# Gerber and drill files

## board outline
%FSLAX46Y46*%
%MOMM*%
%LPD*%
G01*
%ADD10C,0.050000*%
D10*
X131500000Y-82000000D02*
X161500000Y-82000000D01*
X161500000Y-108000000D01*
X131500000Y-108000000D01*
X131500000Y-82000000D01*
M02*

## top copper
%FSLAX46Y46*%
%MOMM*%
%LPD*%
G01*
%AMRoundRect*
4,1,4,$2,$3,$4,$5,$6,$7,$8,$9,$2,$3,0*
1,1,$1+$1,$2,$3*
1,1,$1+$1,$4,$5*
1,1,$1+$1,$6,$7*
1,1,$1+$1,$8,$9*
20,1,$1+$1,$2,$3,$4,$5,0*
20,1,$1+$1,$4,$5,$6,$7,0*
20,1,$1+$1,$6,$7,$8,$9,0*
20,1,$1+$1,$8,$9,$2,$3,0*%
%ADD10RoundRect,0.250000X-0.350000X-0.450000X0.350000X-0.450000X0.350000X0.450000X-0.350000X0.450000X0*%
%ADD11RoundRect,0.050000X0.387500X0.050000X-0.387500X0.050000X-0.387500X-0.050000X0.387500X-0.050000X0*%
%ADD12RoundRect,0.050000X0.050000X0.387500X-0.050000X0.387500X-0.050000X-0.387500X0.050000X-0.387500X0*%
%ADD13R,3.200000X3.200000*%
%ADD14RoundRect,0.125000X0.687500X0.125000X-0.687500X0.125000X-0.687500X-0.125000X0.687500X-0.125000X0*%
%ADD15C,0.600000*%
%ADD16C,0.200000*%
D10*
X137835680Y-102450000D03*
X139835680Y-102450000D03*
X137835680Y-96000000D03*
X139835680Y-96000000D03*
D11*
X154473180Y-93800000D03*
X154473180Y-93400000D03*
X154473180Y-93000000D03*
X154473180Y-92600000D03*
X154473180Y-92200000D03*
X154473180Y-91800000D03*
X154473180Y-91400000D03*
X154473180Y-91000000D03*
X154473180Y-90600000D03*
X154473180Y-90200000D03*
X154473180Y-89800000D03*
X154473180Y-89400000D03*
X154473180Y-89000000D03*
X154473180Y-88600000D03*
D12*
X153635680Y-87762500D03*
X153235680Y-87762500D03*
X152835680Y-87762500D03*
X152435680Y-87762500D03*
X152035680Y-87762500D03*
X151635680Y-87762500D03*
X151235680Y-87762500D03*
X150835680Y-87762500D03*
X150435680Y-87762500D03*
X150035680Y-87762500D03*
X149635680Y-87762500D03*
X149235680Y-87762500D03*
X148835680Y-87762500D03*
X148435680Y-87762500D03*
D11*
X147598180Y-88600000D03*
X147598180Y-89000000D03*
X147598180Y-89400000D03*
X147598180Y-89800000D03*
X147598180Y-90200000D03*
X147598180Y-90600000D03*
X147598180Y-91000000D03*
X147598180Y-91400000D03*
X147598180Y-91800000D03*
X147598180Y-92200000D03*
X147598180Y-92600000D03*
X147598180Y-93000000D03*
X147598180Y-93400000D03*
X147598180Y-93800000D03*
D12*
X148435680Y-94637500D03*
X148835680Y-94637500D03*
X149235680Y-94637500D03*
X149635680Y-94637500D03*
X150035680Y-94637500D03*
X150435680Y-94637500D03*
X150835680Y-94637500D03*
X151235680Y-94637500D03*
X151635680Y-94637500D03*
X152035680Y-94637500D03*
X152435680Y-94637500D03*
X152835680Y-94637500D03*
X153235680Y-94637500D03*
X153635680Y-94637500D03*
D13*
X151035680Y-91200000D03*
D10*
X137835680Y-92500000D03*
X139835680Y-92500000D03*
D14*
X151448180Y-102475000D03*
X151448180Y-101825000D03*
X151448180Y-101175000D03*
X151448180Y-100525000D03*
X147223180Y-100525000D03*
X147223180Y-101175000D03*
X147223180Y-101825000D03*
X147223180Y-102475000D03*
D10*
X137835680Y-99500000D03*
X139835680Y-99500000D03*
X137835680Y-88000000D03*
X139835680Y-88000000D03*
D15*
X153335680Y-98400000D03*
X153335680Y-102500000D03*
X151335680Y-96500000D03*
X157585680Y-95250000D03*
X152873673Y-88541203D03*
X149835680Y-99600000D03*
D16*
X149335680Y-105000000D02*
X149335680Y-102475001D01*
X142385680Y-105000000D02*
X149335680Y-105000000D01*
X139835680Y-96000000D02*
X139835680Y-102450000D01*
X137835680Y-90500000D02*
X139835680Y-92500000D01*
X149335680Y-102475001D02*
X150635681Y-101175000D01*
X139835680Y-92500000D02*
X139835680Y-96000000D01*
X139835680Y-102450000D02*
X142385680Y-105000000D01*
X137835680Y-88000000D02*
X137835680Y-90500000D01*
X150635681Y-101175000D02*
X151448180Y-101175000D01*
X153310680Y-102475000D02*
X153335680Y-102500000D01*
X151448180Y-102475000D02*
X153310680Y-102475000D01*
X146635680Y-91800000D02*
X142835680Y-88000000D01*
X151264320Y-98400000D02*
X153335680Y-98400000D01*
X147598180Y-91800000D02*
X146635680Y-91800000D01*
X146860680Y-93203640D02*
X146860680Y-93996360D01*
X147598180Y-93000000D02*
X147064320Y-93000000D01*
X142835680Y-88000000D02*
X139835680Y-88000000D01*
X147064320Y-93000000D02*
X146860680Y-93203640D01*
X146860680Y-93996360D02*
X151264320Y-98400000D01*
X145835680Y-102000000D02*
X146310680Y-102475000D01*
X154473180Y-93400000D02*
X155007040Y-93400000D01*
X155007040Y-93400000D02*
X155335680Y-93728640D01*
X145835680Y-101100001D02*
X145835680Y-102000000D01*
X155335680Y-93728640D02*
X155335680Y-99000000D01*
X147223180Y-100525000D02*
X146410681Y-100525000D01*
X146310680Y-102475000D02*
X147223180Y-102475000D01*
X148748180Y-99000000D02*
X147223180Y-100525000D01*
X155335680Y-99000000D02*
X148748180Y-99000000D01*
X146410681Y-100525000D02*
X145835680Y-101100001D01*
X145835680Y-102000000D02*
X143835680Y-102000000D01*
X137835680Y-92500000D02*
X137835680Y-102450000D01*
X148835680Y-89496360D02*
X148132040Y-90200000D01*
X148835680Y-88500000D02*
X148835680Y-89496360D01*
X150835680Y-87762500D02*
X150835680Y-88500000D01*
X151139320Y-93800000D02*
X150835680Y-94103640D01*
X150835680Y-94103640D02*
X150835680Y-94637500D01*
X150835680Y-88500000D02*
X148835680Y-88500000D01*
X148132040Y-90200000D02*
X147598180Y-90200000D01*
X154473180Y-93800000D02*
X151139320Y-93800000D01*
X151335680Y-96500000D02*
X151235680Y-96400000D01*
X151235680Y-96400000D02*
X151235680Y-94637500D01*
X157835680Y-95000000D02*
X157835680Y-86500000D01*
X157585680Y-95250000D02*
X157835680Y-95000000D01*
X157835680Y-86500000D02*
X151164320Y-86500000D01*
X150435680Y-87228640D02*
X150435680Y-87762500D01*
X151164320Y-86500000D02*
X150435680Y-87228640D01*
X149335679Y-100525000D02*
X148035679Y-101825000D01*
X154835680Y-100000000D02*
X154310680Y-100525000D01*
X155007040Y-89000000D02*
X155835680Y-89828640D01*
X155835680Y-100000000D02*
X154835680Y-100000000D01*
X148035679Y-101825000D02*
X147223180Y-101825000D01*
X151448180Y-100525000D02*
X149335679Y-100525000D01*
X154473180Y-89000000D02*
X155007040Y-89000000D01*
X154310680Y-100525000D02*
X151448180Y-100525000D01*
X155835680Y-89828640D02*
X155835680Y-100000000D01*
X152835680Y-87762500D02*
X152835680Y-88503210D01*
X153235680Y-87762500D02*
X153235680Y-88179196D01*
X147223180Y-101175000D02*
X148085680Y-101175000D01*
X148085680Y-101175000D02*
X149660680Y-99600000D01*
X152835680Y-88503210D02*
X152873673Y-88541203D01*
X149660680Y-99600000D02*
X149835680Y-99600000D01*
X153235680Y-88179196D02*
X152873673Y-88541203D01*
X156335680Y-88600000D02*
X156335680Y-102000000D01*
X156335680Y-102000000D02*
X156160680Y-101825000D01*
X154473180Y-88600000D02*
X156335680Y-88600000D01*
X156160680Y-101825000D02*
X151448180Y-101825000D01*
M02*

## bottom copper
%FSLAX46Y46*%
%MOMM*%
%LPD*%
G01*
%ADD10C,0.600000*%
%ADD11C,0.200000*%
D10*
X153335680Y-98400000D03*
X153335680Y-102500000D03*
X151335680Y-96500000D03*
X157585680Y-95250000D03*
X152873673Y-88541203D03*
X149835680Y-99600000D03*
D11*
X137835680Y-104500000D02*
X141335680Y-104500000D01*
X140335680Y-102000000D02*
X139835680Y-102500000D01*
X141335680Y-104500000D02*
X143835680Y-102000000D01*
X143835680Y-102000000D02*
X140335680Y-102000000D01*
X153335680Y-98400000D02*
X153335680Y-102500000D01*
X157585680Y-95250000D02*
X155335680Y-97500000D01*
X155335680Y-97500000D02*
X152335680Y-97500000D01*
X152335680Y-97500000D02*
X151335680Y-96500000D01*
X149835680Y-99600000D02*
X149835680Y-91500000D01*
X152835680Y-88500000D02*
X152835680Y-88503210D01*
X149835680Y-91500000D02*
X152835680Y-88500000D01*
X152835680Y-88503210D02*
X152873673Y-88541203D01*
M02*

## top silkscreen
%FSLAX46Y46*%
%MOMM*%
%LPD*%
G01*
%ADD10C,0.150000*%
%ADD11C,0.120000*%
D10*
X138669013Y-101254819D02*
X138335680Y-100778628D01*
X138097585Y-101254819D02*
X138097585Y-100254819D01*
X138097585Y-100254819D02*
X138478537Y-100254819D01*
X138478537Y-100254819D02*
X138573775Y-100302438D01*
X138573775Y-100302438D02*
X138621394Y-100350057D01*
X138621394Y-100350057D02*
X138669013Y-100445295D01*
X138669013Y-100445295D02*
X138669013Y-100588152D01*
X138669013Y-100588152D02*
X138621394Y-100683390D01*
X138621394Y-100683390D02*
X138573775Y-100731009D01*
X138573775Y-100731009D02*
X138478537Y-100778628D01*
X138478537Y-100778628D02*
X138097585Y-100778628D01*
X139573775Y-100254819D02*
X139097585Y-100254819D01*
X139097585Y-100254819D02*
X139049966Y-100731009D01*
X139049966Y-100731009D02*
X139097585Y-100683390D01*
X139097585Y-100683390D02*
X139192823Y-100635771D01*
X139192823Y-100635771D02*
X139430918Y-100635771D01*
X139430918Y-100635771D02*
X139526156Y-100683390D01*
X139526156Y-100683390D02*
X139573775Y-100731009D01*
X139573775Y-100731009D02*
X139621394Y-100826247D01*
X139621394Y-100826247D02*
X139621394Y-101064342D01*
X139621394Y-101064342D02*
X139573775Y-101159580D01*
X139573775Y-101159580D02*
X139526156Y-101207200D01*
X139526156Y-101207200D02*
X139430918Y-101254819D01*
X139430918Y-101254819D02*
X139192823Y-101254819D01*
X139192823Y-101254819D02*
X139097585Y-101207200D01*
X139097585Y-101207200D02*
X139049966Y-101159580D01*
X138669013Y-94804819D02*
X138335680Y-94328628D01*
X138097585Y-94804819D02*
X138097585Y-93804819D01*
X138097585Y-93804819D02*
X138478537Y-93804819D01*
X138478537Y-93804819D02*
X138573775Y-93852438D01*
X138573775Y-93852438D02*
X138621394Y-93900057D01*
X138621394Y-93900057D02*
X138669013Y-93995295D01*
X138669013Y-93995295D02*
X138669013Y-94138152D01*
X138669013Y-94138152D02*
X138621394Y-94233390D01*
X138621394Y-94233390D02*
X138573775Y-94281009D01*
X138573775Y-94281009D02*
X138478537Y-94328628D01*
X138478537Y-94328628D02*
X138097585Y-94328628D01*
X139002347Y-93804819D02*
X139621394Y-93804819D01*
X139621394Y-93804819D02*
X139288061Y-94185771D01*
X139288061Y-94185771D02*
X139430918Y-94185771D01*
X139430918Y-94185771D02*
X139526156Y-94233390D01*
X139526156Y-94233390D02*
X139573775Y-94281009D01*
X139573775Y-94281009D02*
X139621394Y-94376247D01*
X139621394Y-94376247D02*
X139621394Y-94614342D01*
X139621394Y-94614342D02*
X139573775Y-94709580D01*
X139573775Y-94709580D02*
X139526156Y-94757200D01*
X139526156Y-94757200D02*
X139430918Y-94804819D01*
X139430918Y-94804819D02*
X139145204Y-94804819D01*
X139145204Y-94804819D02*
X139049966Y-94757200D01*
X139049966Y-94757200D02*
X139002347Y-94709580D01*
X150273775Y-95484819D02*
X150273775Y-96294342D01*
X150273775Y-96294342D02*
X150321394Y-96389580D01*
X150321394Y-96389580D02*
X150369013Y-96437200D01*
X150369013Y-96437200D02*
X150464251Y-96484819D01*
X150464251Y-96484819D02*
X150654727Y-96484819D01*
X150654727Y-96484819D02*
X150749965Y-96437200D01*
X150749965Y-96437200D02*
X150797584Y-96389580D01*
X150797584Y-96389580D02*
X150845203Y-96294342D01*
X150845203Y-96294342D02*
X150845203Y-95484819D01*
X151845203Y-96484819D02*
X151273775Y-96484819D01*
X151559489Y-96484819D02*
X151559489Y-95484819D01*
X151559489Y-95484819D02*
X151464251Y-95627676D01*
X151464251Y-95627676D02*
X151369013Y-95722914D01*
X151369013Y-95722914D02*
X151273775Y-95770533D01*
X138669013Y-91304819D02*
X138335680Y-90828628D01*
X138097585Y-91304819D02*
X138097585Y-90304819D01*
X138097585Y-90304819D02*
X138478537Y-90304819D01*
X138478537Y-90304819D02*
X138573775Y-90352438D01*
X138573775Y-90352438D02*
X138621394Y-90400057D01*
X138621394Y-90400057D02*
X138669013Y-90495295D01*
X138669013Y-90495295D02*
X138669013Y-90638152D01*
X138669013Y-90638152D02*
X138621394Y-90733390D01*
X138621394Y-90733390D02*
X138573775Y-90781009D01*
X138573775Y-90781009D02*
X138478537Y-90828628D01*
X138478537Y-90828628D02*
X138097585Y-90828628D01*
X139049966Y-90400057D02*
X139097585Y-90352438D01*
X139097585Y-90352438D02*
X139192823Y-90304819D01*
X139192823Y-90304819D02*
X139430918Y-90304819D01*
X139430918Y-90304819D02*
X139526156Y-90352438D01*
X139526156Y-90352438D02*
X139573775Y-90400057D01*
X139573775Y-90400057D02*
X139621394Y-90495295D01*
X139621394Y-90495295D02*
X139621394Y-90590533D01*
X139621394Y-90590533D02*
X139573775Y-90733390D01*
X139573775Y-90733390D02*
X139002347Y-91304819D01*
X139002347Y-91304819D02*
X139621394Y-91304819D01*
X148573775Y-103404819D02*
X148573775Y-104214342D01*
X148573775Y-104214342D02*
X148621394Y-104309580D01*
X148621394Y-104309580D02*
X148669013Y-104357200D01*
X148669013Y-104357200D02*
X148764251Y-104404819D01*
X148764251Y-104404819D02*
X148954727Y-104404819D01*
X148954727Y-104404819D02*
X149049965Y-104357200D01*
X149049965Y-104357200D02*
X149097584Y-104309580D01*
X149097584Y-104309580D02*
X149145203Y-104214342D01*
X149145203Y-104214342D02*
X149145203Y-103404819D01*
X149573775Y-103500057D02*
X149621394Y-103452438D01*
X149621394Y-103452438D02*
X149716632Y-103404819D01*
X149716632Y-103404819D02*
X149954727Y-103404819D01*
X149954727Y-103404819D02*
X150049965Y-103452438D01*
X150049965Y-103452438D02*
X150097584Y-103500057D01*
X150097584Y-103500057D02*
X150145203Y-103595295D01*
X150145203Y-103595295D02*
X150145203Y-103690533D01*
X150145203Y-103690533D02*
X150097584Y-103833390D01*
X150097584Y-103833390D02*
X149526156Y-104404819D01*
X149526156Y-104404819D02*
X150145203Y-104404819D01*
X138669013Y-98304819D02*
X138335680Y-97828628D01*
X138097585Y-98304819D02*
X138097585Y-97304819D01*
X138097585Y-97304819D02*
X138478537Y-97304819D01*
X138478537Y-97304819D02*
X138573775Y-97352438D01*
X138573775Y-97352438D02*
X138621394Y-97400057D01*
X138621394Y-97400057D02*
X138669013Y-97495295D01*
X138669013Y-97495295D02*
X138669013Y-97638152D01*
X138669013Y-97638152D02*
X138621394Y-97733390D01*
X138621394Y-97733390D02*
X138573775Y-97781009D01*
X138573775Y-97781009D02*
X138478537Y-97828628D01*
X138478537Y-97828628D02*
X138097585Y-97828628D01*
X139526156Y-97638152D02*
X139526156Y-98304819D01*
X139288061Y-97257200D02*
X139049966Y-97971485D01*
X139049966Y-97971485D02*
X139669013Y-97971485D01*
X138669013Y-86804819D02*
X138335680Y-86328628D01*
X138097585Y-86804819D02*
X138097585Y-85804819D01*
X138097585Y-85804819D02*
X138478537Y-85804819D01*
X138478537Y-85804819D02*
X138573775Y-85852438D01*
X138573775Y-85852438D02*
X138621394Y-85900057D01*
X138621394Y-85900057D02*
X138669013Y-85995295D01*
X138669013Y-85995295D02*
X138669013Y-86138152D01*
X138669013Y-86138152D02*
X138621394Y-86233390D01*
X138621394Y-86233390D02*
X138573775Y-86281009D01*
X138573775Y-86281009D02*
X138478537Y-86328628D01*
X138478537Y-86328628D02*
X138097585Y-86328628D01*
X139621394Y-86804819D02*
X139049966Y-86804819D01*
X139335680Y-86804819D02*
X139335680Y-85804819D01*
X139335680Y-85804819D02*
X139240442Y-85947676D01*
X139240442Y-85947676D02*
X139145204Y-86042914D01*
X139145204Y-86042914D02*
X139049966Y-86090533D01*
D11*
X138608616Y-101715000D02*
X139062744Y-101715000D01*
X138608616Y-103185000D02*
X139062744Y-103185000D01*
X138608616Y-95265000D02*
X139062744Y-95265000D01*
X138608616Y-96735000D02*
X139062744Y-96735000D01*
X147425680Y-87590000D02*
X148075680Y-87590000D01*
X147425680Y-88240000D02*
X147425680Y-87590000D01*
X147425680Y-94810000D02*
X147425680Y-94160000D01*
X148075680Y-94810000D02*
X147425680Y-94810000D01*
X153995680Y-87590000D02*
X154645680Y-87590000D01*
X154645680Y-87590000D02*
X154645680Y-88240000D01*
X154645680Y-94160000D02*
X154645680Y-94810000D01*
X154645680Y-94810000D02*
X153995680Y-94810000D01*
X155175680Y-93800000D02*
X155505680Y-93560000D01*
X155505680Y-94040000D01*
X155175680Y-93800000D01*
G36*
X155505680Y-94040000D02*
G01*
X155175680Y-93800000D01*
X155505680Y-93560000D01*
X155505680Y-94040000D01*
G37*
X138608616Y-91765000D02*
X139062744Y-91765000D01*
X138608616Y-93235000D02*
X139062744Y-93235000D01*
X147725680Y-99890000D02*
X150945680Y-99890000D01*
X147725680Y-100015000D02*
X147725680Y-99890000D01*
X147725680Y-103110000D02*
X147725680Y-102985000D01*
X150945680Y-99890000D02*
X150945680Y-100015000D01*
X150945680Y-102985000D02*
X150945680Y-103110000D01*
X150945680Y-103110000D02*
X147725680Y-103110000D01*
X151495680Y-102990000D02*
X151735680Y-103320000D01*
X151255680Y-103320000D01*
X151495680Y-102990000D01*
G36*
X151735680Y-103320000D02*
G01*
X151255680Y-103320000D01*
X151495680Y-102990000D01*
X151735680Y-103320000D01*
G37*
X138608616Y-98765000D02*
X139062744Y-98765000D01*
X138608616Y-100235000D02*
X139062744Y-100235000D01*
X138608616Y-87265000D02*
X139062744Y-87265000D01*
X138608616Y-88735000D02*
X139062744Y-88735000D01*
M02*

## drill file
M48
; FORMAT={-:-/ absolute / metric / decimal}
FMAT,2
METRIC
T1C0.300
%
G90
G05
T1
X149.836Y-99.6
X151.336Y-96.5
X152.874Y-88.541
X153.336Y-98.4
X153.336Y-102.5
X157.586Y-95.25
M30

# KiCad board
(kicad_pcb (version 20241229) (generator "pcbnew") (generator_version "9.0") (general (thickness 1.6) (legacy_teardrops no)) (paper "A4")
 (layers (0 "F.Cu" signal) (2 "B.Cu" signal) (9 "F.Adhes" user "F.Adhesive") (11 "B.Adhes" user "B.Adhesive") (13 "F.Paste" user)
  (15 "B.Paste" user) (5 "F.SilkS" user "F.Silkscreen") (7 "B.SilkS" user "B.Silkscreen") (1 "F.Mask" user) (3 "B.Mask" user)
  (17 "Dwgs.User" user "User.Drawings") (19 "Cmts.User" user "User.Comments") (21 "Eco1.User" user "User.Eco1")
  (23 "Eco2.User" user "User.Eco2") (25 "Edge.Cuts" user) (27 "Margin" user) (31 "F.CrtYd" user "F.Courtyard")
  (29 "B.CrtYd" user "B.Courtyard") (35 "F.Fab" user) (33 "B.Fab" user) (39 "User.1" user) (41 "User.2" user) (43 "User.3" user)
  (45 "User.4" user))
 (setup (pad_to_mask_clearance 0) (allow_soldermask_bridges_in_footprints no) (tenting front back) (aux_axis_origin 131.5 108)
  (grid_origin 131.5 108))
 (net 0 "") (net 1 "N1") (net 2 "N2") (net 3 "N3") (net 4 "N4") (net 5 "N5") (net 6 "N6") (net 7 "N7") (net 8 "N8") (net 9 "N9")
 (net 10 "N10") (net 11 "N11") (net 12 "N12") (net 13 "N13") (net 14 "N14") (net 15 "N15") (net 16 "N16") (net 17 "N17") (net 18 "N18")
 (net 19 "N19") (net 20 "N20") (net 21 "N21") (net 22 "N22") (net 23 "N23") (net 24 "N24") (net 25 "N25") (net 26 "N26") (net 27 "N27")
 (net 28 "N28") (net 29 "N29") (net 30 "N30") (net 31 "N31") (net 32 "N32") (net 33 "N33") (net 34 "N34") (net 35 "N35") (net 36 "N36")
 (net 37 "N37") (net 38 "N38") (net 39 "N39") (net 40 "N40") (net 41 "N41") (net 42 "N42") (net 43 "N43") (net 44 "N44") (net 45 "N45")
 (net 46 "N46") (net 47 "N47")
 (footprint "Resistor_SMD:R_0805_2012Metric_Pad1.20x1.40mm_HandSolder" (layer "F.Cu") (at 138.83568 102.45)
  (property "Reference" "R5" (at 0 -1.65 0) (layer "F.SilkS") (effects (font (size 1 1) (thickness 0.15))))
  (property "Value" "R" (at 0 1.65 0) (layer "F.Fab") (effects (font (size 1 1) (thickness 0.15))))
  (fp_line (start -0.227064 -0.735) (end 0.227064 -0.735) (stroke (width 0.12) (type solid)) (layer "F.SilkS"))
  (fp_line (start -0.227064 0.735) (end 0.227064 0.735) (stroke (width 0.12) (type solid)) (layer "F.SilkS"))
  (pad "1" smd roundrect (at -1 0) (size 1.2 1.4) (layers "F.Cu" "F.Mask" "F.Paste") (roundrect_rratio 0.208333) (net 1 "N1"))
  (pad "2" smd roundrect (at 1 0) (size 1.2 1.4) (layers "F.Cu" "F.Mask" "F.Paste") (roundrect_rratio 0.208333) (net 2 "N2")))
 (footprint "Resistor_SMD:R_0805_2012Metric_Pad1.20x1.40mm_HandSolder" (layer "F.Cu") (at 138.83568 96)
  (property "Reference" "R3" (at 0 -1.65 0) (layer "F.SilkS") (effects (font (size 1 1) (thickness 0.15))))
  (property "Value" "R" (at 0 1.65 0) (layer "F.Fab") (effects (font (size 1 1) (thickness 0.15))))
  (fp_line (start -0.227064 -0.735) (end 0.227064 -0.735) (stroke (width 0.12) (type solid)) (layer "F.SilkS"))
  (fp_line (start -0.227064 0.735) (end 0.227064 0.735) (stroke (width 0.12) (type solid)) (layer "F.SilkS"))
  (pad "1" smd roundrect (at -1 0) (size 1.2 1.4) (layers "F.Cu" "F.Mask" "F.Paste") (roundrect_rratio 0.208333) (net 1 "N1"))
  (pad "2" smd roundrect (at 1 0) (size 1.2 1.4) (layers "F.Cu" "F.Mask" "F.Paste") (roundrect_rratio 0.208333) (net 2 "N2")))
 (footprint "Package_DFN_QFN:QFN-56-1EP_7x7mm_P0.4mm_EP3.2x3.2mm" (layer "F.Cu") (at 151.03568 91.2 180)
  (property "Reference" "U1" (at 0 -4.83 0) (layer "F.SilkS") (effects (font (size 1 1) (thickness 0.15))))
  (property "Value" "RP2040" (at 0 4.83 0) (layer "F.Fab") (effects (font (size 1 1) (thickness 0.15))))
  (fp_line (start 3.61 3.61) (end 2.96 3.61) (stroke (width 0.12) (type solid)) (layer "F.SilkS"))
  (fp_line (start 3.61 2.96) (end 3.61 3.61) (stroke (width 0.12) (type solid)) (layer "F.SilkS"))
  (fp_line (start 3.61 -3.61) (end 3.61 -2.96) (stroke (width 0.12) (type solid)) (layer "F.SilkS"))
  (fp_line (start 2.96 -3.61) (end 3.61 -3.61) (stroke (width 0.12) (type solid)) (layer "F.SilkS"))
  (fp_line (start -2.96 3.61) (end -3.61 3.61) (stroke (width 0.12) (type solid)) (layer "F.SilkS"))
  (fp_line (start -3.61 3.61) (end -3.61 2.96) (stroke (width 0.12) (type solid)) (layer "F.SilkS"))
  (fp_line (start -3.61 -2.96) (end -3.61 -3.61) (stroke (width 0.12) (type solid)) (layer "F.SilkS"))
  (fp_line (start -3.61 -3.61) (end -2.96 -3.61) (stroke (width 0.12) (type solid)) (layer "F.SilkS"))
  (fp_poly (pts (xy -4.14 -2.6) (xy -4.47 -2.36) (xy -4.47 -2.84)) (stroke (width 0.12) (type solid)) (fill yes) (layer "F.SilkS"))
  (pad "" smd roundrect (at -0.8 -0.8 180) (size 1.29 1.29) (layers "F.Paste") (roundrect_rratio 0.193798))
  (pad "" smd roundrect (at -0.8 0.8 180) (size 1.29 1.29) (layers "F.Paste") (roundrect_rratio 0.193798))
  (pad "" smd roundrect (at 0.8 -0.8 180) (size 1.29 1.29) (layers "F.Paste") (roundrect_rratio 0.193798))
  (pad "" smd roundrect (at 0.8 0.8 180) (size 1.29 1.29) (layers "F.Paste") (roundrect_rratio 0.193798))
  (pad "1" smd roundrect (at -3.4375 -2.6 180) (size 0.875 0.2) (layers "F.Cu" "F.Mask" "F.Paste") (roundrect_rratio 0.25) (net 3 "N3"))
  (pad "2" smd roundrect (at -3.4375 -2.2 180) (size 0.875 0.2) (layers "F.Cu" "F.Mask" "F.Paste") (roundrect_rratio 0.25) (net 1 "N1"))
  (pad "3" smd roundrect (at -3.4375 -1.8 180) (size 0.875 0.2) (layers "F.Cu" "F.Mask" "F.Paste") (roundrect_rratio 0.25) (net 1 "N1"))
  (pad "4" smd roundrect (at -3.4375 -1.4 180) (size 0.875 0.2) (layers "F.Cu" "F.Mask" "F.Paste") (roundrect_rratio 0.25) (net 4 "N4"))
  (pad "5" smd roundrect (at -3.4375 -1 180) (size 0.875 0.2) (layers "F.Cu" "F.Mask" "F.Paste") (roundrect_rratio 0.25) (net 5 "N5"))
  (pad "6" smd roundrect (at -3.4375 -0.6 180) (size 0.875 0.2) (layers "F.Cu" "F.Mask" "F.Paste") (roundrect_rratio 0.25) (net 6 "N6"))
  (pad "7" smd roundrect (at -3.4375 -0.2 180) (size 0.875 0.2) (layers "F.Cu" "F.Mask" "F.Paste") (roundrect_rratio 0.25) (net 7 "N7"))
  (pad "8" smd roundrect (at -3.4375 0.2 180) (size 0.875 0.2) (layers "F.Cu" "F.Mask" "F.Paste") (roundrect_rratio 0.25) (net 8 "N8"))
  (pad "9" smd roundrect (at -3.4375 0.6 180) (size 0.875 0.2) (layers "F.Cu" "F.Mask" "F.Paste") (roundrect_rratio 0.25) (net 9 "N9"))
  (pad "10" smd roundrect (at -3.4375 1 180) (size 0.875 0.2) (layers "F.Cu" "F.Mask" "F.Paste") (roundrect_rratio 0.25) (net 3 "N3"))
  (pad "11" smd roundrect (at -3.4375 1.4 180) (size 0.875 0.2) (layers "F.Cu" "F.Mask" "F.Paste") (roundrect_rratio 0.25) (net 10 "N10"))
  (pad "12" smd roundrect (at -3.4375 1.8 180) (size 0.875 0.2) (layers "F.Cu" "F.Mask" "F.Paste") (roundrect_rratio 0.25) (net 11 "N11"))
  (pad "13" smd roundrect (at -3.4375 2.2 180) (size 0.875 0.2) (layers "F.Cu" "F.Mask" "F.Paste") (roundrect_rratio 0.25) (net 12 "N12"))
  (pad "14" smd roundrect (at -3.4375 2.6 180) (size 0.875 0.2) (layers "F.Cu" "F.Mask" "F.Paste") (roundrect_rratio 0.25) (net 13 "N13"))
  (pad "15" smd roundrect (at -2.6 3.4375 180) (size 0.2 0.875) (layers "F.Cu" "F.Mask" "F.Paste") (roundrect_rratio 0.25) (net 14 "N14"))
  (pad "16" smd roundrect (at -2.2 3.4375 180) (size 0.2 0.875) (layers "F.Cu" "F.Mask" "F.Paste") (roundrect_rratio 0.25) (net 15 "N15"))
  (pad "17" smd roundrect (at -1.8 3.4375 180) (size 0.2 0.875) (layers "F.Cu" "F.Mask" "F.Paste") (roundrect_rratio 0.25) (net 15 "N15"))
  (pad "18" smd roundrect (at -1.4 3.4375 180) (size 0.2 0.875) (layers "F.Cu" "F.Mask" "F.Paste") (roundrect_rratio 0.25) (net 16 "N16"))
  (pad "19" smd roundrect (at -1 3.4375 180) (size 0.2 0.875) (layers "F.Cu" "F.Mask" "F.Paste") (roundrect_rratio 0.25) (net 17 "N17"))
  (pad "20" smd roundrect (at -0.6 3.4375 180) (size 0.2 0.875) (layers "F.Cu" "F.Mask" "F.Paste") (roundrect_rratio 0.25) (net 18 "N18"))
  (pad "21" smd roundrect (at -0.2 3.4375 180) (size 0.2 0.875) (layers "F.Cu" "F.Mask" "F.Paste") (roundrect_rratio 0.25) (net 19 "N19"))
  (pad "22" smd roundrect (at 0.2 3.4375 180) (size 0.2 0.875) (layers "F.Cu" "F.Mask" "F.Paste") (roundrect_rratio 0.25) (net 3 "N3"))
  (pad "23" smd roundrect (at 0.6 3.4375 180) (size 0.2 0.875) (layers "F.Cu" "F.Mask" "F.Paste") (roundrect_rratio 0.25) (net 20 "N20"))
  (pad "24" smd roundrect (at 1 3.4375 180) (size 0.2 0.875) (layers "F.Cu" "F.Mask" "F.Paste") (roundrect_rratio 0.25) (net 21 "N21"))
  (pad "25" smd roundrect (at 1.4 3.4375 180) (size 0.2 0.875) (layers "F.Cu" "F.Mask" "F.Paste") (roundrect_rratio 0.25) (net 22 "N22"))
  (pad "26" smd roundrect (at 1.8 3.4375 180) (size 0.2 0.875) (layers "F.Cu" "F.Mask" "F.Paste") (roundrect_rratio 0.25) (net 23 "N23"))
  (pad "27" smd roundrect (at 2.2 3.4375 180) (size 0.2 0.875) (layers "F.Cu" "F.Mask" "F.Paste") (roundrect_rratio 0.25) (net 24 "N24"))
  (pad "28" smd roundrect (at 2.6 3.4375 180) (size 0.2 0.875) (layers "F.Cu" "F.Mask" "F.Paste") (roundrect_rratio 0.25) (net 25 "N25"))
  (pad "29" smd roundrect (at 3.4375 2.6 180) (size 0.875 0.2) (layers "F.Cu" "F.Mask" "F.Paste") (roundrect_rratio 0.25) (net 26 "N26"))
  (pad "30" smd roundrect (at 3.4375 2.2 180) (size 0.875 0.2) (layers "F.Cu" "F.Mask" "F.Paste") (roundrect_rratio 0.25) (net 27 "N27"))
  (pad "31" smd roundrect (at 3.4375 1.8 180) (size 0.875 0.2) (layers "F.Cu" "F.Mask" "F.Paste") (roundrect_rratio 0.25) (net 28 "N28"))
  (pad "32" smd roundrect (at 3.4375 1.4 180) (size 0.875 0.2) (layers "F.Cu" "F.Mask" "F.Paste") (roundrect_rratio 0.25) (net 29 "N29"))
  (pad "33" smd roundrect (at 3.4375 1 180) (size 0.875 0.2) (layers "F.Cu" "F.Mask" "F.Paste") (roundrect_rratio 0.25) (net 3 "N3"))
  (pad "34" smd roundrect (at 3.4375 0.6 180) (size 0.875 0.2) (layers "F.Cu" "F.Mask" "F.Paste") (roundrect_rratio 0.25) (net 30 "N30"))
  (pad "35" smd roundrect (at 3.4375 0.2 180) (size 0.875 0.2) (layers "F.Cu" "F.Mask" "F.Paste") (roundrect_rratio 0.25) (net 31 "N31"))
  (pad "36" smd roundrect (at 3.4375 -0.2 180) (size 0.875 0.2) (layers "F.Cu" "F.Mask" "F.Paste") (roundrect_rratio 0.25) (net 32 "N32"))
  (pad "37" smd roundrect (at 3.4375 -0.6 180) (size 0.875 0.2) (layers "F.Cu" "F.Mask" "F.Paste") (roundrect_rratio 0.25) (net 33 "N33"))
  (pad "38" smd roundrect (at 3.4375 -1 180) (size 0.875 0.2) (layers "F.Cu" "F.Mask" "F.Paste") (roundrect_rratio 0.25) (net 33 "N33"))
  (pad "39" smd roundrect (at 3.4375 -1.4 180) (size 0.875 0.2) (layers "F.Cu" "F.Mask" "F.Paste") (roundrect_rratio 0.25) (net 33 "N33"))
  (pad "40" smd roundrect (at 3.4375 -1.8 180) (size 0.875 0.2) (layers "F.Cu" "F.Mask" "F.Paste") (roundrect_rratio 0.25) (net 33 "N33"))
  (pad "41" smd roundrect (at 3.4375 -2.2 180) (size 0.875 0.2) (layers "F.Cu" "F.Mask" "F.Paste") (roundrect_rratio 0.25) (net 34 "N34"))
  (pad "42" smd roundrect (at 3.4375 -2.6 180) (size 0.875 0.2) (layers "F.Cu" "F.Mask" "F.Paste") (roundrect_rratio 0.25) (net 3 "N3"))
  (pad "43" smd roundrect (at 2.6 -3.4375 180) (size 0.2 0.875) (layers "F.Cu" "F.Mask" "F.Paste") (roundrect_rratio 0.25) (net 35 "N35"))
  (pad "44" smd roundrect (at 2.2 -3.4375 180) (size 0.2 0.875) (layers "F.Cu" "F.Mask" "F.Paste") (roundrect_rratio 0.25) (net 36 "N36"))
  (pad "45" smd roundrect (at 1.8 -3.4375 180) (size 0.2 0.875) (layers "F.Cu" "F.Mask" "F.Paste") (roundrect_rratio 0.25) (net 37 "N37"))
  (pad "46" smd roundrect (at 1.4 -3.4375 180) (size 0.2 0.875) (layers "F.Cu" "F.Mask" "F.Paste") (roundrect_rratio 0.25) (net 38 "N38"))
  (pad "47" smd roundrect (at 1 -3.4375 180) (size 0.2 0.875) (layers "F.Cu" "F.Mask" "F.Paste") (roundrect_rratio 0.25) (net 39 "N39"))
  (pad "48" smd roundrect (at 0.6 -3.4375 180) (size 0.2 0.875) (layers "F.Cu" "F.Mask" "F.Paste") (roundrect_rratio 0.25) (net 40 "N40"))
  (pad "49" smd roundrect (at 0.2 -3.4375 180) (size 0.2 0.875) (layers "F.Cu" "F.Mask" "F.Paste") (roundrect_rratio 0.25) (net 3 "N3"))
  (pad "50" smd roundrect (at -0.2 -3.4375 180) (size 0.2 0.875) (layers "F.Cu" "F.Mask" "F.Paste") (roundrect_rratio 0.25) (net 20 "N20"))
  (pad "51" smd roundrect (at -0.6 -3.4375 180) (size 0.2 0.875) (layers "F.Cu" "F.Mask" "F.Paste") (roundrect_rratio 0.25) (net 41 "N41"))
  (pad "52" smd roundrect (at -1 -3.4375 180) (size 0.2 0.875) (layers "F.Cu" "F.Mask" "F.Paste") (roundrect_rratio 0.25) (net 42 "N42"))
  (pad "53" smd roundrect (at -1.4 -3.4375 180) (size 0.2 0.875) (layers "F.Cu" "F.Mask" "F.Paste") (roundrect_rratio 0.25) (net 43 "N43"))
  (pad "54" smd roundrect (at -1.8 -3.4375 180) (size 0.2 0.875) (layers "F.Cu" "F.Mask" "F.Paste") (roundrect_rratio 0.25) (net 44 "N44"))
  (pad "55" smd roundrect (at -2.2 -3.4375 180) (size 0.2 0.875) (layers "F.Cu" "F.Mask" "F.Paste") (roundrect_rratio 0.25) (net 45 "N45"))
  (pad "56" smd roundrect (at -2.6 -3.4375 180) (size 0.2 0.875) (layers "F.Cu" "F.Mask" "F.Paste") (roundrect_rratio 0.25) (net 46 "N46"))
  (pad "57" smd rect (at 0 0 180) (size 3.2 3.2) (layers "F.Cu" "F.Mask") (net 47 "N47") (zone_connect 2)))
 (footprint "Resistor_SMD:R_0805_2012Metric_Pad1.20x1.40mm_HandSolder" (layer "F.Cu") (at 138.83568 92.5)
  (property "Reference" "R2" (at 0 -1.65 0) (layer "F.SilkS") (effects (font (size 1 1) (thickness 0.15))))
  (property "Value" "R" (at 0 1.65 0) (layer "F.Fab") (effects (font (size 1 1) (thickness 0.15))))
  (fp_line (start -0.227064 -0.735) (end 0.227064 -0.735) (stroke (width 0.12) (type solid)) (layer "F.SilkS"))
  (fp_line (start -0.227064 0.735) (end 0.227064 0.735) (stroke (width 0.12) (type solid)) (layer "F.SilkS"))
  (pad "1" smd roundrect (at -1 0) (size 1.2 1.4) (layers "F.Cu" "F.Mask" "F.Paste") (roundrect_rratio 0.208333) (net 1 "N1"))
  (pad "2" smd roundrect (at 1 0) (size 1.2 1.4) (layers "F.Cu" "F.Mask" "F.Paste") (roundrect_rratio 0.208333) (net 2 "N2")))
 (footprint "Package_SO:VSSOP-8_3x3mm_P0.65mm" (layer "F.Cu") (at 149.33568 101.5 180)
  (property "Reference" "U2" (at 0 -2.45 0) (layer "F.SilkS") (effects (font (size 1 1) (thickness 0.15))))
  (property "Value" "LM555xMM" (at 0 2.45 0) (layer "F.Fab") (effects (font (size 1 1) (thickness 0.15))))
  (fp_line (start 1.61 1.61) (end -1.61 1.61) (stroke (width 0.12) (type solid)) (layer "F.SilkS"))
  (fp_line (start 1.61 1.485) (end 1.61 1.61) (stroke (width 0.12) (type solid)) (layer "F.SilkS"))
  (fp_line (start 1.61 -1.61) (end 1.61 -1.485) (stroke (width 0.12) (type solid)) (layer "F.SilkS"))
  (fp_line (start -1.61 1.61) (end -1.61 1.485) (stroke (width 0.12) (type solid)) (layer "F.SilkS"))
  (fp_line (start -1.61 -1.485) (end -1.61 -1.61) (stroke (width 0.12) (type solid)) (layer "F.SilkS"))
  (fp_line (start -1.61 -1.61) (end 1.61 -1.61) (stroke (width 0.12) (type solid)) (layer "F.SilkS"))
  (fp_poly (pts (xy -2.16 -1.49) (xy -2.4 -1.82) (xy -1.92 -1.82)) (stroke (width 0.12) (type solid)) (fill yes) (layer "F.SilkS"))
  (pad "1" smd roundrect (at -2.1125 -0.975 180) (size 1.625 0.5) (layers "F.Cu" "F.Mask" "F.Paste") (roundrect_rratio 0.25) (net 33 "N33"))
  (pad "2" smd roundrect (at -2.1125 -0.325 180) (size 1.625 0.5) (layers "F.Cu" "F.Mask" "F.Paste") (roundrect_rratio 0.25) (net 13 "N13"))
  (pad "3" smd roundrect (at -2.1125 0.325 180) (size 1.625 0.5) (layers "F.Cu" "F.Mask" "F.Paste") (roundrect_rratio 0.25) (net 2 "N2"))
  (pad "4" smd roundrect (at -2.1125 0.975 180) (size 1.625 0.5) (layers "F.Cu" "F.Mask" "F.Paste") (roundrect_rratio 0.25) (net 12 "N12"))
  (pad "5" smd roundrect (at 2.1125 0.975 180) (size 1.625 0.5) (layers "F.Cu" "F.Mask" "F.Paste") (roundrect_rratio 0.25) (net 1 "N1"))
  (pad "6" smd roundrect (at 2.1125 0.325 180) (size 1.625 0.5) (layers "F.Cu" "F.Mask" "F.Paste") (roundrect_rratio 0.25) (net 15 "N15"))
  (pad "7" smd roundrect (at 2.1125 -0.325 180) (size 1.625 0.5) (layers "F.Cu" "F.Mask" "F.Paste") (roundrect_rratio 0.25) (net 12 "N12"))
  (pad "8" smd roundrect (at 2.1125 -0.975 180) (size 1.625 0.5) (layers "F.Cu" "F.Mask" "F.Paste") (roundrect_rratio 0.25) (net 1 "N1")))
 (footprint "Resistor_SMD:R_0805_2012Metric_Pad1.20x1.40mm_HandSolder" (layer "F.Cu") (at 138.83568 99.5)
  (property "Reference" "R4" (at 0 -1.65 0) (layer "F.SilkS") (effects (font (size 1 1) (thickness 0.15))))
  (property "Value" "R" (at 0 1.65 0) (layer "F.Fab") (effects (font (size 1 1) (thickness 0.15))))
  (fp_line (start -0.227064 -0.735) (end 0.227064 -0.735) (stroke (width 0.12) (type solid)) (layer "F.SilkS"))
  (fp_line (start -0.227064 0.735) (end 0.227064 0.735) (stroke (width 0.12) (type solid)) (layer "F.SilkS"))
  (pad "1" smd roundrect (at -1 0) (size 1.2 1.4) (layers "F.Cu" "F.Mask" "F.Paste") (roundrect_rratio 0.208333) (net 1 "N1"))
  (pad "2" smd roundrect (at 1 0) (size 1.2 1.4) (layers "F.Cu" "F.Mask" "F.Paste") (roundrect_rratio 0.208333) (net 2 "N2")))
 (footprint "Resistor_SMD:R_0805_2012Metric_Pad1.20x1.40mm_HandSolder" (layer "F.Cu") (at 138.83568 88)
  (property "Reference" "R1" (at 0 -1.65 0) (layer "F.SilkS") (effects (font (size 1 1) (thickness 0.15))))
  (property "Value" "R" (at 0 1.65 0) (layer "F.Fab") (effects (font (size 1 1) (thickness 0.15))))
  (fp_line (start -0.227064 -0.735) (end 0.227064 -0.735) (stroke (width 0.12) (type solid)) (layer "F.SilkS"))
  (fp_line (start -0.227064 0.735) (end 0.227064 0.735) (stroke (width 0.12) (type solid)) (layer "F.SilkS"))
  (pad "1" smd roundrect (at -1 0) (size 1.2 1.4) (layers "F.Cu" "F.Mask" "F.Paste") (roundrect_rratio 0.208333) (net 2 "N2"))
  (pad "2" smd roundrect (at 1 0) (size 1.2 1.4) (layers "F.Cu" "F.Mask" "F.Paste") (roundrect_rratio 0.208333) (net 33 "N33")))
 (gr_rect (start 131.5 82) (end 161.5 108) (stroke (width 0.05) (type default)) (fill no) (layer "Edge.Cuts"))
 (segment (start 137.83568 104.5) (end 141.33568 104.5) (width 0.2) (layer "B.Cu") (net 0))
 (segment (start 140.33568 102) (end 139.83568 102.5) (width 0.2) (layer "B.Cu") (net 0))
 (segment (start 141.33568 104.5) (end 143.83568 102) (width 0.2) (layer "B.Cu") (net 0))
 (segment (start 143.83568 102) (end 140.33568 102) (width 0.2) (layer "B.Cu") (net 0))
 (segment (start 149.33568 105) (end 149.33568 102.475001) (width 0.2) (layer "F.Cu") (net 2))
 (segment (start 142.38568 105) (end 149.33568 105) (width 0.2) (layer "F.Cu") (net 2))
 (segment (start 139.83568 96) (end 139.83568 102.45) (width 0.2) (layer "F.Cu") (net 2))
 (segment (start 137.83568 90.5) (end 139.83568 92.5) (width 0.2) (layer "F.Cu") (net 2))
 (segment (start 149.33568 102.475001) (end 150.635681 101.175) (width 0.2) (layer "F.Cu") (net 2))
 (segment (start 139.83568 92.5) (end 139.83568 96) (width 0.2) (layer "F.Cu") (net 2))
 (segment (start 139.83568 102.45) (end 142.38568 105) (width 0.2) (layer "F.Cu") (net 2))
 (segment (start 137.83568 88) (end 137.83568 90.5) (width 0.2) (layer "F.Cu") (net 2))
 (segment (start 150.635681 101.175) (end 151.44818 101.175) (width 0.2) (layer "F.Cu") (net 2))
 (segment (start 153.31068 102.475) (end 153.33568 102.5) (width 0.2) (layer "F.Cu") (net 33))
 (segment (start 151.44818 102.475) (end 153.31068 102.475) (width 0.2) (layer "F.Cu") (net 33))
 (segment (start 146.63568 91.8) (end 142.83568 88) (width 0.2) (layer "F.Cu") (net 33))
 (segment (start 151.26432 98.4) (end 153.33568 98.4) (width 0.2) (layer "F.Cu") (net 33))
 (segment (start 147.59818 91.8) (end 146.63568 91.8) (width 0.2) (layer "F.Cu") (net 33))
 (segment (start 146.86068 93.20364) (end 146.86068 93.99636) (width 0.2) (layer "F.Cu") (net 33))
 (segment (start 147.59818 93) (end 147.06432 93) (width 0.2) (layer "F.Cu") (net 33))
 (segment (start 142.83568 88) (end 139.83568 88) (width 0.2) (layer "F.Cu") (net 33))
 (segment (start 147.06432 93) (end 146.86068 93.20364) (width 0.2) (layer "F.Cu") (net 33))
 (segment (start 146.86068 93.99636) (end 151.26432 98.4) (width 0.2) (layer "F.Cu") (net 33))
 (via (at 153.33568 98.4) (size 0.6) (drill 0.3) (layers "F.Cu" "B.Cu") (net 33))
 (via (at 153.33568 102.5) (size 0.6) (drill 0.3) (layers "F.Cu" "B.Cu") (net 33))
 (segment (start 153.33568 98.4) (end 153.33568 102.5) (width 0.2) (layer "B.Cu") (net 33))
 (segment (start 145.83568 102) (end 146.31068 102.475) (width 0.2) (layer "F.Cu") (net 1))
 (segment (start 154.47318 93.4) (end 155.00704 93.4) (width 0.2) (layer "F.Cu") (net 1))
 (segment (start 155.00704 93.4) (end 155.33568 93.72864) (width 0.2) (layer "F.Cu") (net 1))
 (segment (start 145.83568 101.100001) (end 145.83568 102) (width 0.2) (layer "F.Cu") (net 1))
 (segment (start 155.33568 93.72864) (end 155.33568 99) (width 0.2) (layer "F.Cu") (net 1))
 (segment (start 147.22318 100.525) (end 146.410681 100.525) (width 0.2) (layer "F.Cu") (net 1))
 (segment (start 146.31068 102.475) (end 147.22318 102.475) (width 0.2) (layer "F.Cu") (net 1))
 (segment (start 148.74818 99) (end 147.22318 100.525) (width 0.2) (layer "F.Cu") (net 1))
 (segment (start 155.33568 99) (end 148.74818 99) (width 0.2) (layer "F.Cu") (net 1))
 (segment (start 146.410681 100.525) (end 145.83568 101.100001) (width 0.2) (layer "F.Cu") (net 1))
 (segment (start 145.83568 102) (end 143.83568 102) (width 0.2) (layer "F.Cu") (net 1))
 (segment (start 137.83568 92.5) (end 137.83568 102.45) (width 0.2) (layer "F.Cu") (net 1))
 (segment (start 148.83568 89.49636) (end 148.13204 90.2) (width 0.2) (layer "F.Cu") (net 3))
 (segment (start 148.83568 88.5) (end 148.83568 89.49636) (width 0.2) (layer "F.Cu") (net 3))
 (segment (start 150.83568 87.7625) (end 150.83568 88.5) (width 0.2) (layer "F.Cu") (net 3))
 (segment (start 151.13932 93.8) (end 150.83568 94.10364) (width 0.2) (layer "F.Cu") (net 3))
 (segment (start 150.83568 94.10364) (end 150.83568 94.6375) (width 0.2) (layer "F.Cu") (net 3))
 (segment (start 150.83568 88.5) (end 148.83568 88.5) (width 0.2) (layer "F.Cu") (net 3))
 (segment (start 148.13204 90.2) (end 147.59818 90.2) (width 0.2) (layer "F.Cu") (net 3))
 (segment (start 154.47318 93.8) (end 151.13932 93.8) (width 0.2) (layer "F.Cu") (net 3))
 (segment (start 151.33568 96.5) (end 151.23568 96.4) (width 0.2) (layer "F.Cu") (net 20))
 (segment (start 151.23568 96.4) (end 151.23568 94.6375) (width 0.2) (layer "F.Cu") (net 20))
 (segment (start 157.83568 95) (end 157.83568 86.5) (width 0.2) (layer "F.Cu") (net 20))
 (segment (start 157.58568 95.25) (end 157.83568 95) (width 0.2) (layer "F.Cu") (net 20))
 (segment (start 157.83568 86.5) (end 151.16432 86.5) (width 0.2) (layer "F.Cu") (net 20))
 (segment (start 150.43568 87.22864) (end 150.43568 87.7625) (width 0.2) (layer "F.Cu") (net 20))
 (segment (start 151.16432 86.5) (end 150.43568 87.22864) (width 0.2) (layer "F.Cu") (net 20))
 (via (at 151.33568 96.5) (size 0.6) (drill 0.3) (layers "F.Cu" "B.Cu") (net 20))
 (via (at 157.58568 95.25) (size 0.6) (drill 0.3) (layers "F.Cu" "B.Cu") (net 20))
 (segment (start 157.58568 95.25) (end 155.33568 97.5) (width 0.2) (layer "B.Cu") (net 20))
 (segment (start 155.33568 97.5) (end 152.33568 97.5) (width 0.2) (layer "B.Cu") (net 20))
 (segment (start 152.33568 97.5) (end 151.33568 96.5) (width 0.2) (layer "B.Cu") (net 20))
 (segment (start 149.335679 100.525) (end 148.035679 101.825) (width 0.2) (layer "F.Cu") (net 12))
 (segment (start 154.83568 100) (end 154.31068 100.525) (width 0.2) (layer "F.Cu") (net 12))
 (segment (start 155.00704 89) (end 155.83568 89.82864) (width 0.2) (layer "F.Cu") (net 12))
 (segment (start 155.83568 100) (end 154.83568 100) (width 0.2) (layer "F.Cu") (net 12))
 (segment (start 148.035679 101.825) (end 147.22318 101.825) (width 0.2) (layer "F.Cu") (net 12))
 (segment (start 151.44818 100.525) (end 149.335679 100.525) (width 0.2) (layer "F.Cu") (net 12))
 (segment (start 154.47318 89) (end 155.00704 89) (width 0.2) (layer "F.Cu") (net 12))
 (segment (start 154.31068 100.525) (end 151.44818 100.525) (width 0.2) (layer "F.Cu") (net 12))
 (segment (start 155.83568 89.82864) (end 155.83568 100) (width 0.2) (layer "F.Cu") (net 12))
 (segment (start 152.83568 87.7625) (end 152.83568 88.50321) (width 0.2) (layer "F.Cu") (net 15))
 (segment (start 153.23568 87.7625) (end 153.23568 88.179196) (width 0.2) (layer "F.Cu") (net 15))
 (segment (start 147.22318 101.175) (end 148.08568 101.175) (width 0.2) (layer "F.Cu") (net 15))
 (segment (start 148.08568 101.175) (end 149.66068 99.6) (width 0.2) (layer "F.Cu") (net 15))
 (segment (start 152.83568 88.50321) (end 152.873673 88.541203) (width 0.2) (layer "F.Cu") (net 15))
 (segment (start 149.66068 99.6) (end 149.83568 99.6) (width 0.2) (layer "F.Cu") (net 15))
 (segment (start 153.23568 88.179196) (end 152.873673 88.541203) (width 0.2) (layer "F.Cu") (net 15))
 (via (at 152.873673 88.541203) (size 0.6) (drill 0.3) (layers "F.Cu" "B.Cu") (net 15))
 (via (at 149.83568 99.6) (size 0.6) (drill 0.3) (layers "F.Cu" "B.Cu") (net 15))
 (segment (start 149.83568 99.6) (end 149.83568 91.5) (width 0.2) (layer "B.Cu") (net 15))
 (segment (start 152.83568 88.5) (end 152.83568 88.50321) (width 0.2) (layer "B.Cu") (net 15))
 (segment (start 149.83568 91.5) (end 152.83568 88.5) (width 0.2) (layer "B.Cu") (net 15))
 (segment (start 152.83568 88.50321) (end 152.873673 88.541203) (width 0.2) (layer "B.Cu") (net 15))
 (segment (start 156.33568 88.6) (end 156.33568 102) (width 0.2) (layer "F.Cu") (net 13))
 (segment (start 156.33568 102) (end 156.16068 101.825) (width 0.2) (layer "F.Cu") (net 13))
 (segment (start 154.47318 88.6) (end 156.33568 88.6) (width 0.2) (layer "F.Cu") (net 13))
 (segment (start 156.16068 101.825) (end 151.44818 101.825) (width 0.2) (layer "F.Cu") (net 13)))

